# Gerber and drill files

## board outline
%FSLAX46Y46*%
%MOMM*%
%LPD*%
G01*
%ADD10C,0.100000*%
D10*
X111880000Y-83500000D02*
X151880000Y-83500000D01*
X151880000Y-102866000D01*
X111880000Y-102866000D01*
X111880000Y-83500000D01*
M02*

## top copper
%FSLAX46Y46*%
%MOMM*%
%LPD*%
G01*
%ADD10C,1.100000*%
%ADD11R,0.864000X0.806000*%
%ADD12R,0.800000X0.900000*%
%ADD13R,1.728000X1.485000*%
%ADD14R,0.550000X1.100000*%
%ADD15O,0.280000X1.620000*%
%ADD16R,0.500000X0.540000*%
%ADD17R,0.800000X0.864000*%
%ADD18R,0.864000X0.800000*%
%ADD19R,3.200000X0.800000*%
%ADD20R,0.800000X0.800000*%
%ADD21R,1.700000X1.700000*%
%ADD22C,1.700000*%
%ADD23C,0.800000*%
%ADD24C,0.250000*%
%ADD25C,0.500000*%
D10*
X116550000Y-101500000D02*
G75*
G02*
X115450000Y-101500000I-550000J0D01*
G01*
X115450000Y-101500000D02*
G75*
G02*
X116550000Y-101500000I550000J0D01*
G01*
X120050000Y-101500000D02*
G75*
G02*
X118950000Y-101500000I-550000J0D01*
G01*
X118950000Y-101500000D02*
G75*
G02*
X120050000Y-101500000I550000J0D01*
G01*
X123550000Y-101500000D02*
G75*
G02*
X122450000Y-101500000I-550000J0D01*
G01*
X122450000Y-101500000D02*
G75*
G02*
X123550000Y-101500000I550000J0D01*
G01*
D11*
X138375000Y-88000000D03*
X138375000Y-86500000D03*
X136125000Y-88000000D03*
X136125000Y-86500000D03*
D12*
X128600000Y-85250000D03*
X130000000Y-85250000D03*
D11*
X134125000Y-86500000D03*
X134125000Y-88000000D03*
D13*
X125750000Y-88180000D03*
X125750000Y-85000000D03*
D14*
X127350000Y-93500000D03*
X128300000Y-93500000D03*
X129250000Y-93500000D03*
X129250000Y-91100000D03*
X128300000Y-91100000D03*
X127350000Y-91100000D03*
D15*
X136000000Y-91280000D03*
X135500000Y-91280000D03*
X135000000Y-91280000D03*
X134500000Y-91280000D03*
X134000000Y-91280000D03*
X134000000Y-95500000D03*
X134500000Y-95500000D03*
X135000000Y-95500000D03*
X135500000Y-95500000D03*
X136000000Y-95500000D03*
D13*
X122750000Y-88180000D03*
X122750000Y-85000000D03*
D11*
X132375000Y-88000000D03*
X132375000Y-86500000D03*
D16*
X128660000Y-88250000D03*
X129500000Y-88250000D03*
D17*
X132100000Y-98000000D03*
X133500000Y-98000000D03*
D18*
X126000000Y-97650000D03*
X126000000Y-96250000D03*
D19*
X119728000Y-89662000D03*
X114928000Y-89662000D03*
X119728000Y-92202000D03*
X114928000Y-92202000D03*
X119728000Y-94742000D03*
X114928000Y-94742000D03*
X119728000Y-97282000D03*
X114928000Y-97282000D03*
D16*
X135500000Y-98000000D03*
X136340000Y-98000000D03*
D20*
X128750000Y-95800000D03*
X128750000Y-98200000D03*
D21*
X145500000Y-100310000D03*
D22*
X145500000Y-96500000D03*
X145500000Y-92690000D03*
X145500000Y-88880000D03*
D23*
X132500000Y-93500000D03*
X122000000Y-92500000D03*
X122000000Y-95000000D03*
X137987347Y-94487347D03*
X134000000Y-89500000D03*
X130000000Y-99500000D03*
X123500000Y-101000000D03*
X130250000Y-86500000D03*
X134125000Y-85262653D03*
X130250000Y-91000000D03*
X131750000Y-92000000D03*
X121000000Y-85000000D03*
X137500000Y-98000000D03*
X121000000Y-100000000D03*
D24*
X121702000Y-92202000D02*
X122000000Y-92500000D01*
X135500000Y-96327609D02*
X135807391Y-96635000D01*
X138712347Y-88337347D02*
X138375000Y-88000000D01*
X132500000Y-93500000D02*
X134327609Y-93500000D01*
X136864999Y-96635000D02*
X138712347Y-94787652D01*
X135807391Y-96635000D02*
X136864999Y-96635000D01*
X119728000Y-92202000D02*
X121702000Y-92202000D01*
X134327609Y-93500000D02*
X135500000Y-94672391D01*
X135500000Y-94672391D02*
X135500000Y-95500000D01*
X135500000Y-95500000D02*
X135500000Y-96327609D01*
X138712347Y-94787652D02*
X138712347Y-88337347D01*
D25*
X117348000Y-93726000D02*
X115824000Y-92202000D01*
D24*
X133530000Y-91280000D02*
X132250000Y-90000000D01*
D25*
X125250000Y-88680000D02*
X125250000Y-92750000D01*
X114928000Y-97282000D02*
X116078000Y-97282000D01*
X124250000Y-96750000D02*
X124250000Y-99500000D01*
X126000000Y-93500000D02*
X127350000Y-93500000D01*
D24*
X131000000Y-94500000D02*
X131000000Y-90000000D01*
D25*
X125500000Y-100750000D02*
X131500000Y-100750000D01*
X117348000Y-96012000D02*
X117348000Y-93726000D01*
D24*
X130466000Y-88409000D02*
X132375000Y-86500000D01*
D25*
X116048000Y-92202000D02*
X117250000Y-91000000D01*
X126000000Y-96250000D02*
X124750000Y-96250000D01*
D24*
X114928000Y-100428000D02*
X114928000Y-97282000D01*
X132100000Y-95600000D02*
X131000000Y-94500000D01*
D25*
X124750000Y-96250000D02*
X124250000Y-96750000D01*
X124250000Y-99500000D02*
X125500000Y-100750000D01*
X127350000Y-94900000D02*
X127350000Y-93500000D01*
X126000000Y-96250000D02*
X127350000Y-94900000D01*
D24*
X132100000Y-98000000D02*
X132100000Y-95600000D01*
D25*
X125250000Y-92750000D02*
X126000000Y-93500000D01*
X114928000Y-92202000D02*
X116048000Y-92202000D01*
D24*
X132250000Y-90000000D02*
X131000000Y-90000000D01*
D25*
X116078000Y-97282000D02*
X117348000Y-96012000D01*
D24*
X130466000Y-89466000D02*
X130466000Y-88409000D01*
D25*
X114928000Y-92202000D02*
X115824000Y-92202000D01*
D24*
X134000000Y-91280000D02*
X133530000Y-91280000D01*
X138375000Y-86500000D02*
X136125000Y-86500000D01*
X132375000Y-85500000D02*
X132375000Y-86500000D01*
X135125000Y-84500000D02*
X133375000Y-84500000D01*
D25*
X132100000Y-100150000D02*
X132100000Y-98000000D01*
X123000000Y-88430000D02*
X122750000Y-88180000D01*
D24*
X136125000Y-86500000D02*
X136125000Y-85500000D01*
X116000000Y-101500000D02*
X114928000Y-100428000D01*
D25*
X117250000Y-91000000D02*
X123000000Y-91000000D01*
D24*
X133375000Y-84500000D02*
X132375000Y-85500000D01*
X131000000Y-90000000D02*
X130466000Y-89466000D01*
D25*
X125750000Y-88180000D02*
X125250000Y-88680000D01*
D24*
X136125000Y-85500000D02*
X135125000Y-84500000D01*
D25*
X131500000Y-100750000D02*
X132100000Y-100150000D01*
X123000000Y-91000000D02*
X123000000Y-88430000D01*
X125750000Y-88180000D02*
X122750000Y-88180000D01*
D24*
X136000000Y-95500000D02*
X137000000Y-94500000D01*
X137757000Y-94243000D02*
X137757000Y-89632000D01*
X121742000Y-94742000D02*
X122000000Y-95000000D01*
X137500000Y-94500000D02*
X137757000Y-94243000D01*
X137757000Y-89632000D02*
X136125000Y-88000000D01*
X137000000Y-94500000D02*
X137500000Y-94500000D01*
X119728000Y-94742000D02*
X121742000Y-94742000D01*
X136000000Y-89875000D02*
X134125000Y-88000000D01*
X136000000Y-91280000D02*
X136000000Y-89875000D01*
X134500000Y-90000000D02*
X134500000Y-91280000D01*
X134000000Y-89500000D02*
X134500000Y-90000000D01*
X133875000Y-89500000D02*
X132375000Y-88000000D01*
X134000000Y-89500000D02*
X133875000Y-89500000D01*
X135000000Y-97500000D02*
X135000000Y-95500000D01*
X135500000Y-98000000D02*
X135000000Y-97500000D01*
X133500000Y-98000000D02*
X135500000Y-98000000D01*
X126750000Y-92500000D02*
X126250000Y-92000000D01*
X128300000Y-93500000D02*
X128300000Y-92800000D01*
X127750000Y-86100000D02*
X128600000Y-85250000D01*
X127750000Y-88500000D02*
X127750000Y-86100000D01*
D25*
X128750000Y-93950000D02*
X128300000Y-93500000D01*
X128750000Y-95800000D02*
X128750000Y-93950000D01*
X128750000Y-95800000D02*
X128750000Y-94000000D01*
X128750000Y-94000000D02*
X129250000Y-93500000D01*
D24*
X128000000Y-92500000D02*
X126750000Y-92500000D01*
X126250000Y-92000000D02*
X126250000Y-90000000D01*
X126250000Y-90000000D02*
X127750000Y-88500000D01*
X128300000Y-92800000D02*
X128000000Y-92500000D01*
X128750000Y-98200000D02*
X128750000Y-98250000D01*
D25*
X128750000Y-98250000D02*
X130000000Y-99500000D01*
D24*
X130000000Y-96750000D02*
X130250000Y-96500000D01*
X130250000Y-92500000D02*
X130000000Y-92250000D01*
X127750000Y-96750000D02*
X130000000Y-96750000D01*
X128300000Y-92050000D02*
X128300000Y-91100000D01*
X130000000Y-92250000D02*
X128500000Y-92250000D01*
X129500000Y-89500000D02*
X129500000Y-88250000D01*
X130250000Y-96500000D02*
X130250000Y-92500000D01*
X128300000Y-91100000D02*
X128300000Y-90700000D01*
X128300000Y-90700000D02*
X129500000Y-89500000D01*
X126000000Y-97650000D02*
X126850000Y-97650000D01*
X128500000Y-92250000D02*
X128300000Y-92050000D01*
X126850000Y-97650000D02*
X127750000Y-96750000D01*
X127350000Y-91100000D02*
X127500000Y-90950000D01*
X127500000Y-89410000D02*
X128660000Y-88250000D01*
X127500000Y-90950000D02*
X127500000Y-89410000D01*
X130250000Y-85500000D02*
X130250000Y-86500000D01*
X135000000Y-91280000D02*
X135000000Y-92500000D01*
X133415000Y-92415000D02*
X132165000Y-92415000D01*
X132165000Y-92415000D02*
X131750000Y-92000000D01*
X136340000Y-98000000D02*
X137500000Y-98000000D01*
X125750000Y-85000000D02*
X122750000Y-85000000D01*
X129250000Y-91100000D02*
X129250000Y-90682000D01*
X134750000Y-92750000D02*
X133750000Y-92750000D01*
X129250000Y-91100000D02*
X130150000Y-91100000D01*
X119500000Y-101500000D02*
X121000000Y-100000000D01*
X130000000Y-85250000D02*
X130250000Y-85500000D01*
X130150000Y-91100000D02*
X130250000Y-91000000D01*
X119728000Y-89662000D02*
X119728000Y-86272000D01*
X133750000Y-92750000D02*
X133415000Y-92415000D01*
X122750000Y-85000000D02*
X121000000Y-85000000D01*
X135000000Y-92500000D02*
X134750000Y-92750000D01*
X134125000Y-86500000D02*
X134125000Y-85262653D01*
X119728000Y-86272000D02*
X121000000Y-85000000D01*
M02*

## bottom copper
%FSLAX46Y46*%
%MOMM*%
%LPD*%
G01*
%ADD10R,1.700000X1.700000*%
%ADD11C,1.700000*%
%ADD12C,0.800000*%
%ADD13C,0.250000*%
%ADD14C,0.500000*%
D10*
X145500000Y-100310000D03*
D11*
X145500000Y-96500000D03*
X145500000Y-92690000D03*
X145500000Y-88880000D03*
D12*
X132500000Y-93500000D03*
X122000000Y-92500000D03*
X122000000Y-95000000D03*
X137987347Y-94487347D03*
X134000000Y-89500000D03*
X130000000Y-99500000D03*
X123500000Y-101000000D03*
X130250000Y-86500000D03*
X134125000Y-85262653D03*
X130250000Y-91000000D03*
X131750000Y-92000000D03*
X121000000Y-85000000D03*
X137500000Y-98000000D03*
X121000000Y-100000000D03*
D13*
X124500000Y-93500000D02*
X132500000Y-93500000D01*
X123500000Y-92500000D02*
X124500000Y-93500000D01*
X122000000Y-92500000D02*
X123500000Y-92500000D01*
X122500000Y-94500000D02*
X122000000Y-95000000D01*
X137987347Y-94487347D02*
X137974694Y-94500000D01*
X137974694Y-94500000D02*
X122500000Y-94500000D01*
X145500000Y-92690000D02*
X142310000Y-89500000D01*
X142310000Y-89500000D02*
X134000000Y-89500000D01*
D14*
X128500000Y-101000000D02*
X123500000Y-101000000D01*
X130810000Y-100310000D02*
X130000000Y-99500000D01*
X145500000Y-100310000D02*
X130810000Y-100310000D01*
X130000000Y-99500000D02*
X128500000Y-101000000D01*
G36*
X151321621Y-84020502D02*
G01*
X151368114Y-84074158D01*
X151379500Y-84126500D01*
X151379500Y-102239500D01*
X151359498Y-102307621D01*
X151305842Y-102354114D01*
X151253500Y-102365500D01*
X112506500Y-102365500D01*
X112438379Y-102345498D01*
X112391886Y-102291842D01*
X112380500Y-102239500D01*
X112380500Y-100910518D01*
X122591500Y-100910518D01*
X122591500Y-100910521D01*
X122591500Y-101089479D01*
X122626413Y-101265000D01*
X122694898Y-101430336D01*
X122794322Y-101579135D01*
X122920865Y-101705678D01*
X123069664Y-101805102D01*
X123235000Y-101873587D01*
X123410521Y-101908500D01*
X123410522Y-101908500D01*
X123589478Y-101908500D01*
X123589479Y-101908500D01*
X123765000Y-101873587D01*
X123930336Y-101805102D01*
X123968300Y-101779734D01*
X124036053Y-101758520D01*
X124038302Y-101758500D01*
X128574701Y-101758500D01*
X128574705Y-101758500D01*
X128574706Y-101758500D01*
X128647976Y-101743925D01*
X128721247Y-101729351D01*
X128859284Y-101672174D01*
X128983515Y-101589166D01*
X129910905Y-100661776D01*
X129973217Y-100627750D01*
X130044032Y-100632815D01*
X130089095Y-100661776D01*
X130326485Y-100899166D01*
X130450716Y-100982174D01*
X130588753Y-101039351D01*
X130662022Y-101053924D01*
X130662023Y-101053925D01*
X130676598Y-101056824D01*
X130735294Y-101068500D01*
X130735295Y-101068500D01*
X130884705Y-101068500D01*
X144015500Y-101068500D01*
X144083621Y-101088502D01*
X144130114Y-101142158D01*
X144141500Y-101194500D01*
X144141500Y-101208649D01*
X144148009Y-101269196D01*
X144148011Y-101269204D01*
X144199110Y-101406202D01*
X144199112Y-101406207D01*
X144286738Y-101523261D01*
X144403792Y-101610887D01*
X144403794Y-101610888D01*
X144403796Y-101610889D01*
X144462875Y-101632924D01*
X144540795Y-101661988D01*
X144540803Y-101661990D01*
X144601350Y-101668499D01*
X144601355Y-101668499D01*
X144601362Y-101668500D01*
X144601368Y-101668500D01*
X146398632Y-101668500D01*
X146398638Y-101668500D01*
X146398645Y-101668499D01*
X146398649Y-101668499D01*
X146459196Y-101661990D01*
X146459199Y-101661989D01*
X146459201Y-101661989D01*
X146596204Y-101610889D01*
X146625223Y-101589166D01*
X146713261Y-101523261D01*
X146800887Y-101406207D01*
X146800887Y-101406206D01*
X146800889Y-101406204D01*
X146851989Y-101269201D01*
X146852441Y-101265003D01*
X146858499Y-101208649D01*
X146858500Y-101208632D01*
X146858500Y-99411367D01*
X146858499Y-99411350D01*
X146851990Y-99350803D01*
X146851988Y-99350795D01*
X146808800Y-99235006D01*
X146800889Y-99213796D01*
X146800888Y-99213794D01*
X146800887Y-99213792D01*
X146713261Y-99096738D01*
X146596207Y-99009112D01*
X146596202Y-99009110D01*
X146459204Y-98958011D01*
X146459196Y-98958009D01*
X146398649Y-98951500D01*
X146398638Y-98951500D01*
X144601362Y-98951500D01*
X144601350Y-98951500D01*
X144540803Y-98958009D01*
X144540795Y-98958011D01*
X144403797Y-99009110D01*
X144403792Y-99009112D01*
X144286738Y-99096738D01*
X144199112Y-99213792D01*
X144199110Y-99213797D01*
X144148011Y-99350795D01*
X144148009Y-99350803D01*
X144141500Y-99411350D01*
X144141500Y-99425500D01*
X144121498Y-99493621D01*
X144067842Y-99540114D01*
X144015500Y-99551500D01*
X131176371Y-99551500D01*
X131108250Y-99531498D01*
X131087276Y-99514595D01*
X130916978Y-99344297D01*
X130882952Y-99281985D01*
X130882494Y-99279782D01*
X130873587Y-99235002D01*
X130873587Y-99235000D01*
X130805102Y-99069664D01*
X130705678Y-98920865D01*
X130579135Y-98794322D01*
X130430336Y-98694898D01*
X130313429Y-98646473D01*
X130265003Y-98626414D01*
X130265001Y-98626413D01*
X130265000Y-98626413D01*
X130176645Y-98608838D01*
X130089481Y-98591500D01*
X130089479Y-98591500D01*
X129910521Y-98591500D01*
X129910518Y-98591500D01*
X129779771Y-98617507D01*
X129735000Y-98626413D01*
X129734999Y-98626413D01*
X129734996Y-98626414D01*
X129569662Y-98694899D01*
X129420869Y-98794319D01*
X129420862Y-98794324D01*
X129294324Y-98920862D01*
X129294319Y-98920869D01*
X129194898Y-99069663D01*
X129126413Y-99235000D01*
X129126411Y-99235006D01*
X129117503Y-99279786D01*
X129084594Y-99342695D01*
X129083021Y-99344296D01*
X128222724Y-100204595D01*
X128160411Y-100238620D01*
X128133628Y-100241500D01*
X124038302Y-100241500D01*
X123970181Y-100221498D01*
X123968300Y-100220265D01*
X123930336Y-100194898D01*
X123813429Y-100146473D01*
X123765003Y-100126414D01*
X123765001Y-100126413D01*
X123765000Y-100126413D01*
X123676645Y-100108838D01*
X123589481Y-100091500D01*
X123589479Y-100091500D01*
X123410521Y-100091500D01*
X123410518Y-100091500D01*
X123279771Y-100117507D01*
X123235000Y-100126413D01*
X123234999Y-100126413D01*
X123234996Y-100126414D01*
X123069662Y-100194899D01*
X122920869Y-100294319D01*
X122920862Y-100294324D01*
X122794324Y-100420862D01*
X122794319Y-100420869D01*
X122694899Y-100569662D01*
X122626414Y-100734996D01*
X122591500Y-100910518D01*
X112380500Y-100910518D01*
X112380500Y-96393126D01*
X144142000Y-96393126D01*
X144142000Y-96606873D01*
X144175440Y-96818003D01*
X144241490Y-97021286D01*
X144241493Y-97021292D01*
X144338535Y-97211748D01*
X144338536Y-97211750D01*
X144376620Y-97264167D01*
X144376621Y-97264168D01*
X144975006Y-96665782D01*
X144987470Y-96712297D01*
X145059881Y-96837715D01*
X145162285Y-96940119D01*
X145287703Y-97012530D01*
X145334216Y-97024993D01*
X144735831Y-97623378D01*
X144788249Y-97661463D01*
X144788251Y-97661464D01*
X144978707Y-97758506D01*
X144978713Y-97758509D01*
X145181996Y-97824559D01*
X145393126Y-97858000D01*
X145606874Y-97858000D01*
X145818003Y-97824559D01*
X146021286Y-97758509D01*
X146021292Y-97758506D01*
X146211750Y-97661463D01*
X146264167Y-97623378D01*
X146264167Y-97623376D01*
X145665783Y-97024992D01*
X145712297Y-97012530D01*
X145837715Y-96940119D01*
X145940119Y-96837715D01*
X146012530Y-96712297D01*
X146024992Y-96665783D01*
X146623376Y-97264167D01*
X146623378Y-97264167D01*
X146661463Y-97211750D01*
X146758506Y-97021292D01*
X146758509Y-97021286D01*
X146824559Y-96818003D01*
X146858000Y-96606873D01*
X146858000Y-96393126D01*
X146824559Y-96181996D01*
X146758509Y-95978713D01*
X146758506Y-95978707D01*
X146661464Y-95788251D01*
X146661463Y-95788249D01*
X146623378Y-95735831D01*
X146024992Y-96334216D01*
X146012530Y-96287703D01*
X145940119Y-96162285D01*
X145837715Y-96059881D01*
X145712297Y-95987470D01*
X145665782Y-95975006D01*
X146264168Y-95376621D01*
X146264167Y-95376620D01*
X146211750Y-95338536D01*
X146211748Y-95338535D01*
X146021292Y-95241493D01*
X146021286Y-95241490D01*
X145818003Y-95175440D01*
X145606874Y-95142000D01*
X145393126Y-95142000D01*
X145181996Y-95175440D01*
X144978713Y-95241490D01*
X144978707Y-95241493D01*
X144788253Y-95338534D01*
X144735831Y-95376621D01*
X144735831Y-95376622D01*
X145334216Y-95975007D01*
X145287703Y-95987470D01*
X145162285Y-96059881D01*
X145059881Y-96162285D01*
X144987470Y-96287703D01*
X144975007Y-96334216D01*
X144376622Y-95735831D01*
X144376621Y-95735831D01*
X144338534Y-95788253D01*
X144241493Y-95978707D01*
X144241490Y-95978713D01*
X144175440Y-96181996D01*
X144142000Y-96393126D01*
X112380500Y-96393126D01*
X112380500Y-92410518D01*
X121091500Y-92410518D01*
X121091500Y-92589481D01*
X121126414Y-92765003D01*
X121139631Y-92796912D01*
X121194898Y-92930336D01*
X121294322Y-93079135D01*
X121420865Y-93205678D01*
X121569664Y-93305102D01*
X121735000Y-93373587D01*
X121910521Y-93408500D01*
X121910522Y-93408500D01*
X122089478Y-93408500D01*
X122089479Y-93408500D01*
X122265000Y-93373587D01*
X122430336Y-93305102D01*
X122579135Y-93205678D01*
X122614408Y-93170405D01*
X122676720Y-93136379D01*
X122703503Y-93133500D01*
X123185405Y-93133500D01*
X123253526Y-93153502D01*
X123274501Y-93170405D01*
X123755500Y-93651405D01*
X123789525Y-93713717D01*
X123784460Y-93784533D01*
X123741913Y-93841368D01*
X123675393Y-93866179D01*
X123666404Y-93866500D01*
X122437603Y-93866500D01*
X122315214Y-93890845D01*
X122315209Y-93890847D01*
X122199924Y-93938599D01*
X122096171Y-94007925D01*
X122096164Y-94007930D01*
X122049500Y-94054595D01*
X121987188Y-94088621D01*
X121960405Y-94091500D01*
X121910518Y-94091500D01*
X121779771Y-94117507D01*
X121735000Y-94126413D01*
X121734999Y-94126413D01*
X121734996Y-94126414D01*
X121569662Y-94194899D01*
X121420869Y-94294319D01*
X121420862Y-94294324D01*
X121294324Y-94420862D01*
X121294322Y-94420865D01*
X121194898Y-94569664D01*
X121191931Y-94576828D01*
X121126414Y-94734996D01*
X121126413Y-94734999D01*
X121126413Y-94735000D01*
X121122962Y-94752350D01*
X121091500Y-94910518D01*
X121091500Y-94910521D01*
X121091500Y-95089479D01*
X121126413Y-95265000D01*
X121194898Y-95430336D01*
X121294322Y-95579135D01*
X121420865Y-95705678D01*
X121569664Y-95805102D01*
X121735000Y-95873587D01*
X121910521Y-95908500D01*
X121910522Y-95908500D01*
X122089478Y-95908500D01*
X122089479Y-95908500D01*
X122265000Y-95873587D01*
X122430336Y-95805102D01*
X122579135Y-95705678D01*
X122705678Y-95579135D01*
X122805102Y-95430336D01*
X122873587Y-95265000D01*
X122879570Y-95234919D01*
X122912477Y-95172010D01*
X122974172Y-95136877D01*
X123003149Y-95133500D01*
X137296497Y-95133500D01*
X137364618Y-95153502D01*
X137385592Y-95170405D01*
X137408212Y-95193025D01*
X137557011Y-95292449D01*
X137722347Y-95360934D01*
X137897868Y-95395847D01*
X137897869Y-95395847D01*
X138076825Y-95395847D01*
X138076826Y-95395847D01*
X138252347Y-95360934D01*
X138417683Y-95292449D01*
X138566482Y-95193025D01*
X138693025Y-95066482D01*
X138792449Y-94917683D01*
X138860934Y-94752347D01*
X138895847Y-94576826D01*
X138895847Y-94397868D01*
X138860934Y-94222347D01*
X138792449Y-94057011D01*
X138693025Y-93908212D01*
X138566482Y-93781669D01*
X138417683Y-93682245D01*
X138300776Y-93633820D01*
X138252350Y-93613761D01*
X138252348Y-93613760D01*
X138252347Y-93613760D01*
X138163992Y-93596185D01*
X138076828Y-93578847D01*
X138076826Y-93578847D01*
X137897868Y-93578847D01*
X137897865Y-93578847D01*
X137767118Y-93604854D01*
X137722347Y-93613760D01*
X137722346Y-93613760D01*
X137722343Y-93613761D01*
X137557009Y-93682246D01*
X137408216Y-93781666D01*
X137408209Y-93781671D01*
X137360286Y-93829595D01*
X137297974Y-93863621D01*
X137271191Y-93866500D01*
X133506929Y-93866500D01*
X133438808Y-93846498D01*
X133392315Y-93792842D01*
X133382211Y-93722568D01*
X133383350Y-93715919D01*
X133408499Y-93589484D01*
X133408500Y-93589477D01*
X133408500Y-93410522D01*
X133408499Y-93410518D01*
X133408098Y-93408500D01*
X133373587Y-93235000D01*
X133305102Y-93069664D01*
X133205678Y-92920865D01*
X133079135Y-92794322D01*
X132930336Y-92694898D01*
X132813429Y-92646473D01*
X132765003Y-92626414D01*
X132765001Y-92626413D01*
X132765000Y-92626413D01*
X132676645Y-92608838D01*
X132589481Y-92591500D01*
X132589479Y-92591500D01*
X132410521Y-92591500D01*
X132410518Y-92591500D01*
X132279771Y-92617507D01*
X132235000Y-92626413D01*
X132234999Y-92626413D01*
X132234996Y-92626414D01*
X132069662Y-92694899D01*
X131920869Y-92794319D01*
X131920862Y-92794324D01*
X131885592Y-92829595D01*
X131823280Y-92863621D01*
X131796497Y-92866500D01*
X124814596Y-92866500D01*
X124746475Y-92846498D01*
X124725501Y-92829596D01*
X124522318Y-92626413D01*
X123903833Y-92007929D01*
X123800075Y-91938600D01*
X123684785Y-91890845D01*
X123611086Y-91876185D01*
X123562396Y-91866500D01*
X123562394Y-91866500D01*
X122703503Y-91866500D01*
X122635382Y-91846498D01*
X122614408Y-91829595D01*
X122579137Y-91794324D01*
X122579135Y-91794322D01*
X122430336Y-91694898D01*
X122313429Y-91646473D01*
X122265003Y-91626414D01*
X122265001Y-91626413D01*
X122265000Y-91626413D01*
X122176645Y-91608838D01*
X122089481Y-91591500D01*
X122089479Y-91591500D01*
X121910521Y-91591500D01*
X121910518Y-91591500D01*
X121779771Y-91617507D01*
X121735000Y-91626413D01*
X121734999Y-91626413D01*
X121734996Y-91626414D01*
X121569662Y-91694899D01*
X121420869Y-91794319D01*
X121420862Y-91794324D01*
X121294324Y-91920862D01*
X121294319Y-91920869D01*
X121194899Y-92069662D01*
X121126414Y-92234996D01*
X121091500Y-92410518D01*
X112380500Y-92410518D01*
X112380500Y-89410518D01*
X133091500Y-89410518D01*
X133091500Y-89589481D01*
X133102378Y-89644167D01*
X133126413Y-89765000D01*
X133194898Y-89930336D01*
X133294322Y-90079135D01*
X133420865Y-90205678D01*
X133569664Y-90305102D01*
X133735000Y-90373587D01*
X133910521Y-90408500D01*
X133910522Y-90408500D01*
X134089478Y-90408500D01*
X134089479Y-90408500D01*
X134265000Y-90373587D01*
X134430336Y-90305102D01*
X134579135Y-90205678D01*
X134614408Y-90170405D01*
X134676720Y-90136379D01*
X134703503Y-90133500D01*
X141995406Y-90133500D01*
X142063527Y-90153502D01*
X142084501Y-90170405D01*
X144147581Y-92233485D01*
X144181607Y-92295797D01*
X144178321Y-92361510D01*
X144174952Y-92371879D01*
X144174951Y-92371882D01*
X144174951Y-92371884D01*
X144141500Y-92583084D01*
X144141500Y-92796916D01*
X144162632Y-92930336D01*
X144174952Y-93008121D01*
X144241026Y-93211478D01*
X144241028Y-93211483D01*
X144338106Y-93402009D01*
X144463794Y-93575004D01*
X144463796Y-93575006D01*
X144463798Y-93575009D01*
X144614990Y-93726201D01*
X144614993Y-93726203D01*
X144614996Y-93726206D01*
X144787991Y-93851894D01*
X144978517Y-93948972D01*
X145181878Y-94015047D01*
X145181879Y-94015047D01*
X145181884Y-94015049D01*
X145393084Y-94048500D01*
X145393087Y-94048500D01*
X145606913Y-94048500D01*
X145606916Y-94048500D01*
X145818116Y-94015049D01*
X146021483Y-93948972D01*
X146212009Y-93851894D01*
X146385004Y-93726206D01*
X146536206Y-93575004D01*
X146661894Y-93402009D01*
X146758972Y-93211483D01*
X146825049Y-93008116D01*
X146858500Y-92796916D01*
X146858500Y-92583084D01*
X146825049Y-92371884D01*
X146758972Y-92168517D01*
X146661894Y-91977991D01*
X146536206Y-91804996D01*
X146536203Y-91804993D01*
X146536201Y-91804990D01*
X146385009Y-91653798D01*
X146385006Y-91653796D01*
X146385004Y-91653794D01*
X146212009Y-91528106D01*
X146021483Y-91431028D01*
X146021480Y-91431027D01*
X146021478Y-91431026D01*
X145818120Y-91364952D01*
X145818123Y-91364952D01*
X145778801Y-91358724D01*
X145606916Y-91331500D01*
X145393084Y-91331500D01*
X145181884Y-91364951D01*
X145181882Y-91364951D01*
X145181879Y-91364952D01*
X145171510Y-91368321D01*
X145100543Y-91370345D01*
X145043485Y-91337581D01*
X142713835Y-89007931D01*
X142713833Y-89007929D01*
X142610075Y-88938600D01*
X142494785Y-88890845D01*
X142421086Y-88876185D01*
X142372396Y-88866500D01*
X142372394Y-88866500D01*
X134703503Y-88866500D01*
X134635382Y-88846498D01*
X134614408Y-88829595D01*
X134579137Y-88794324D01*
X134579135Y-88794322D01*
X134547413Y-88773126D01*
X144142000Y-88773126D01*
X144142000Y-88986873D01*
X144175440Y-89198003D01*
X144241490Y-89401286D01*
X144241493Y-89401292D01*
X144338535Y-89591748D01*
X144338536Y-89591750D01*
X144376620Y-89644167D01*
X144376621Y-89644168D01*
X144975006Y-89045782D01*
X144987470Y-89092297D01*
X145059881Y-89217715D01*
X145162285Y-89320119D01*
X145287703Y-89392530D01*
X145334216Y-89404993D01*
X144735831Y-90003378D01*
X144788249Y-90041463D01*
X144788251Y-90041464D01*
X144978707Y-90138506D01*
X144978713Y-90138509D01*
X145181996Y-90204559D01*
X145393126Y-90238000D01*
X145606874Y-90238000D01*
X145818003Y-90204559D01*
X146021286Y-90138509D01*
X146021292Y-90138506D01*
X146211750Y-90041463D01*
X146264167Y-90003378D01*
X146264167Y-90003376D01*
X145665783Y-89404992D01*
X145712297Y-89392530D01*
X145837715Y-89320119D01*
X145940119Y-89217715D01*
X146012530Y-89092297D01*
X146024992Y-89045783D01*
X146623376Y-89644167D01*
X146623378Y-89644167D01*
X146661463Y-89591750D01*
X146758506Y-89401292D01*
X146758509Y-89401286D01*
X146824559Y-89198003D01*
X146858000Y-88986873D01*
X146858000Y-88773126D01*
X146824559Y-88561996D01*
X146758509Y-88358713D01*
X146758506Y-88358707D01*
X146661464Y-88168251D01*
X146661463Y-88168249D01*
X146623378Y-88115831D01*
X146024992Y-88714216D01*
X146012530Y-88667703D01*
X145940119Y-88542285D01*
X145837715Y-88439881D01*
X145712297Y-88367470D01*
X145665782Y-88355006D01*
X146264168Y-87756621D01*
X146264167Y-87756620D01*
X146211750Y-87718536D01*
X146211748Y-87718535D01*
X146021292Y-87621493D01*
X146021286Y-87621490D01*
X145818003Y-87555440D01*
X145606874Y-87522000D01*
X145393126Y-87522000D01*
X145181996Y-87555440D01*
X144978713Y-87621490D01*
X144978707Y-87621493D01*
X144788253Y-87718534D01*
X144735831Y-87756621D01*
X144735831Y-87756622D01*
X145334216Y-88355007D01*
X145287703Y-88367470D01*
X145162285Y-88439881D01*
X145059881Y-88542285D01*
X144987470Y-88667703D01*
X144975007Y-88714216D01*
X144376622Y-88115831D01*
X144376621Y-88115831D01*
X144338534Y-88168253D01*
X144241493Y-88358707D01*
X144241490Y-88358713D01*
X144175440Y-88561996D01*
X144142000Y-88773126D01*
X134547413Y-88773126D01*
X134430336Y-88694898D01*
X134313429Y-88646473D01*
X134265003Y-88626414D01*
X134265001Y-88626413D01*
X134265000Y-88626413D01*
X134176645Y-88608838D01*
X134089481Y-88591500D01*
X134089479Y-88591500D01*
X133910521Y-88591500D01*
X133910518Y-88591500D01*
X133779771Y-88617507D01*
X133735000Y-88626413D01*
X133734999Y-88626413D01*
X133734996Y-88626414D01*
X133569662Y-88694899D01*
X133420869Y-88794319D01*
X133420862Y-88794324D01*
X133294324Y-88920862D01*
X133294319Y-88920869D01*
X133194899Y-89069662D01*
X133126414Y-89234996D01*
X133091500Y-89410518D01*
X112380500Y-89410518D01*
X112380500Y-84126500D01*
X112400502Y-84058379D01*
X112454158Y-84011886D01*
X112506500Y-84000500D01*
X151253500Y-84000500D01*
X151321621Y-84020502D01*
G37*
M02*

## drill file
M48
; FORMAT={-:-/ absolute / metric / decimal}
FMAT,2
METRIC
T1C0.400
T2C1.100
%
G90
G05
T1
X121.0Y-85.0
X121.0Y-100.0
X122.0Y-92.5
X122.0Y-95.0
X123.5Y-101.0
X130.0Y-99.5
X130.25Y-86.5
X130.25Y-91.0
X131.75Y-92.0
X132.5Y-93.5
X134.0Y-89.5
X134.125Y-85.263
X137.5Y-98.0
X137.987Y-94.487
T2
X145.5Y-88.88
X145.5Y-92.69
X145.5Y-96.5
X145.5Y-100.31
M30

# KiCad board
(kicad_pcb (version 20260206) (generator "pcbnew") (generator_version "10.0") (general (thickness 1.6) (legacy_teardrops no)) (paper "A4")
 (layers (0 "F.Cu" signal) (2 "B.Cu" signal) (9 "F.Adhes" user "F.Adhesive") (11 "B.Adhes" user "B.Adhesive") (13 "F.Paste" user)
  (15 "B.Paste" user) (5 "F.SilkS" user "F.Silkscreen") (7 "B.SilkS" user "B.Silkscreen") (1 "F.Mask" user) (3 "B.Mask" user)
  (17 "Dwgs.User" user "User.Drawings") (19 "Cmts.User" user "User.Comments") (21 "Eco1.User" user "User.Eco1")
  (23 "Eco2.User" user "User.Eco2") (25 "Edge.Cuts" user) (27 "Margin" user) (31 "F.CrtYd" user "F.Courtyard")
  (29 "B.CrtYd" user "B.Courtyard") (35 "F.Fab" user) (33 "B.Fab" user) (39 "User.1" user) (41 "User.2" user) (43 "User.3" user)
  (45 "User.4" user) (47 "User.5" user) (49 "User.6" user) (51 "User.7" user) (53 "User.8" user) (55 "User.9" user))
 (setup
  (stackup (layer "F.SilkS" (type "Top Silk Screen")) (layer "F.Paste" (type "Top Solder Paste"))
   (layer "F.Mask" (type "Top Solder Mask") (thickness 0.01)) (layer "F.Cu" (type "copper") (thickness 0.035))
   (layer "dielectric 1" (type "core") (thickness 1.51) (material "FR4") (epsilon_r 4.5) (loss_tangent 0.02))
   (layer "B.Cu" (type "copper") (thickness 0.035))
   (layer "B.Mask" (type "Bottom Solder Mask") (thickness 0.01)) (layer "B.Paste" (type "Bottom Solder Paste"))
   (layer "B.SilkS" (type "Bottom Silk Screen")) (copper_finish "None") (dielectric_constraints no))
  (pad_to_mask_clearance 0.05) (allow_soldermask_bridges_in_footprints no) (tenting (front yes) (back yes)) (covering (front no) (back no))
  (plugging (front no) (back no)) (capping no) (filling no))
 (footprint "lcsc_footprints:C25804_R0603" (layer "F.Cu") (at 138.375 87.25 90)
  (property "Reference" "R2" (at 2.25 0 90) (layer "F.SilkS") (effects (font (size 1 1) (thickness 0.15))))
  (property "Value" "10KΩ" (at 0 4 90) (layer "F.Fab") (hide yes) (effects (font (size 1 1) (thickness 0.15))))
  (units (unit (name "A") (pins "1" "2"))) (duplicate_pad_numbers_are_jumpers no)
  (pad "1" smd rect (at -0.75 0 90) (size 0.806 0.864) (layers "F.Cu" "F.Mask" "F.Paste") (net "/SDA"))
  (pad "2" smd rect (at 0.75 0 90) (size 0.806 0.864) (layers "F.Cu" "F.Mask" "F.Paste") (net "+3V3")))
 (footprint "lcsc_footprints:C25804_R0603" (layer "F.Cu") (at 136.125 87.25 90)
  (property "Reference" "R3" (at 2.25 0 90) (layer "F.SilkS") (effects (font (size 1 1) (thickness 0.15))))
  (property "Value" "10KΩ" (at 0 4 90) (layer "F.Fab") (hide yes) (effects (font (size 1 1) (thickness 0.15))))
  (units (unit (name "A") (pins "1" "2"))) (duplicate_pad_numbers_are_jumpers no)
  (pad "1" smd rect (at -0.75 0 90) (size 0.806 0.864) (layers "F.Cu" "F.Mask" "F.Paste") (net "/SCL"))
  (pad "2" smd rect (at 0.75 0 90) (size 0.806 0.864) (layers "F.Cu" "F.Mask" "F.Paste") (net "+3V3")))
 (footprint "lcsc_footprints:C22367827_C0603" (layer "F.Cu") (at 129.3 85.25)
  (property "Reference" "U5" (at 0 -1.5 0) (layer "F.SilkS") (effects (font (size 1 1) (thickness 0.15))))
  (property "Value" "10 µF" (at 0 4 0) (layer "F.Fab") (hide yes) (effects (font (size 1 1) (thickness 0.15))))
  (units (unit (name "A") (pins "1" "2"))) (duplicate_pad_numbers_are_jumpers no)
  (pad "1" smd rect (at -0.7 0) (size 0.8 0.9) (layers "F.Cu" "F.Mask" "F.Paste") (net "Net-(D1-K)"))
  (pad "2" smd rect (at 0.7 0) (size 0.8 0.9) (layers "F.Cu" "F.Mask" "F.Paste") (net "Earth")))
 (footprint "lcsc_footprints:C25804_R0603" (layer "F.Cu") (at 134.125 87.25 -90)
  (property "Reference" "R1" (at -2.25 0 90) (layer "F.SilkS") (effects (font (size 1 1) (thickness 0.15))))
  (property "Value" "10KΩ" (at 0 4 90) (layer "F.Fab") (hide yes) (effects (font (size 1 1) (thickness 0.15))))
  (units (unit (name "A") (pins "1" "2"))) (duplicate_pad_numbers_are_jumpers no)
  (pad "1" smd rect (at -0.75 0 270) (size 0.806 0.864) (layers "F.Cu" "F.Mask" "F.Paste") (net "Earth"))
  (pad "2" smd rect (at 0.75 0 270) (size 0.806 0.864) (layers "F.Cu" "F.Mask" "F.Paste") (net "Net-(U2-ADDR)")))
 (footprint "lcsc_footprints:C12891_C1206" (layer "F.Cu") (at 125.75 86.59 90)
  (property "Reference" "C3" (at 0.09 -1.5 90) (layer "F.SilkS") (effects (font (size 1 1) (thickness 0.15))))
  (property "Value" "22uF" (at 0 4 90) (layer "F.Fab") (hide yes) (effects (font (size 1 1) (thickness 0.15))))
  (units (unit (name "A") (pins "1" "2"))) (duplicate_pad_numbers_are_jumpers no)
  (pad "1" smd rect (at -1.59 0 90) (size 1.485 1.728) (layers "F.Cu" "F.Mask" "F.Paste") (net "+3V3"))
  (pad "2" smd rect (at 1.59 0 90) (size 1.485 1.728) (layers "F.Cu" "F.Mask" "F.Paste") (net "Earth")))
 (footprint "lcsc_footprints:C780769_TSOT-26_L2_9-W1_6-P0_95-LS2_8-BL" (layer "F.Cu") (at 128.3 92.3)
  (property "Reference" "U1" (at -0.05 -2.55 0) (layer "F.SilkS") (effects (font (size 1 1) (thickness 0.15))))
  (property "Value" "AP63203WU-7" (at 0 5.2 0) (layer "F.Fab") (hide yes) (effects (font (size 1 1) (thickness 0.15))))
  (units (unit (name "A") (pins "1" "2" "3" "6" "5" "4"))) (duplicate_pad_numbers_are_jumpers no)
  (pad "1" smd rect (at -0.95 1.2 180) (size 0.55 1.1) (layers "F.Cu" "F.Mask" "F.Paste") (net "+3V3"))
  (pad "2" smd rect (at 0 1.2 180) (size 0.55 1.1) (layers "F.Cu" "F.Mask" "F.Paste") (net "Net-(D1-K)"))
  (pad "3" smd rect (at 0.95 1.2 180) (size 0.55 1.1) (layers "F.Cu" "F.Mask" "F.Paste") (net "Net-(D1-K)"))
  (pad "4" smd rect (at 0.95 -1.2 180) (size 0.55 1.1) (layers "F.Cu" "F.Mask" "F.Paste") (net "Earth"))
  (pad "5" smd rect (at 0 -1.2 180) (size 0.55 1.1) (layers "F.Cu" "F.Mask" "F.Paste") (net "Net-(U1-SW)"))
  (pad "6" smd rect (at -0.95 -1.2 180) (size 0.55 1.1) (layers "F.Cu" "F.Mask" "F.Paste") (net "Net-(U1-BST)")))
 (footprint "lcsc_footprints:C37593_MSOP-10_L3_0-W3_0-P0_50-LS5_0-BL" (layer "F.Cu") (at 135 93.39 180)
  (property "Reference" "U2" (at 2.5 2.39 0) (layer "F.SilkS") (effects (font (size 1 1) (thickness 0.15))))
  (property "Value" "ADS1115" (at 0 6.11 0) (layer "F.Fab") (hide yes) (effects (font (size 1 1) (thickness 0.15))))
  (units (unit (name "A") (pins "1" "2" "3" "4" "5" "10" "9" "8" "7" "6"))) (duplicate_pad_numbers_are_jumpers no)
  (pad "1" smd oval (at -1 2.11 180) (size 0.28 1.62) (layers "F.Cu" "F.Mask" "F.Paste") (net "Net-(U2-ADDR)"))
  (pad "2" smd oval (at -0.5 2.11 180) (size 0.28 1.62) (layers "F.Cu" "F.Mask" "F.Paste") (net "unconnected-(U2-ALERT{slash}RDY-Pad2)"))
  (pad "3" smd oval (at 0 2.11 180) (size 0.28 1.62) (layers "F.Cu" "F.Mask" "F.Paste") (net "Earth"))
  (pad "4" smd oval (at 0.5 2.11 180) (size 0.28 1.62) (layers "F.Cu" "F.Mask" "F.Paste") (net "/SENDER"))
  (pad "5" smd oval (at 1 2.11 180) (size 0.28 1.62) (layers "F.Cu" "F.Mask" "F.Paste") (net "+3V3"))
  (pad "6" smd oval (at 1 -2.11 180) (size 0.28 1.62) (layers "F.Cu" "F.Mask" "F.Paste") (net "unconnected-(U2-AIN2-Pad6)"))
  (pad "7" smd oval (at 0.5 -2.11 180) (size 0.28 1.62) (layers "F.Cu" "F.Mask" "F.Paste") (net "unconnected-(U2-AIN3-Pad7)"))
  (pad "8" smd oval (at 0 -2.11 180) (size 0.28 1.62) (layers "F.Cu" "F.Mask" "F.Paste") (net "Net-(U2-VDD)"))
  (pad "9" smd oval (at -0.5 -2.11 180) (size 0.28 1.62) (layers "F.Cu" "F.Mask" "F.Paste") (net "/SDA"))
  (pad "10" smd oval (at -1 -2.11 180) (size 0.28 1.62) (layers "F.Cu" "F.Mask" "F.Paste") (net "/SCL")))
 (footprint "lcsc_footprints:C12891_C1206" (layer "F.Cu") (at 122.75 86.59 90)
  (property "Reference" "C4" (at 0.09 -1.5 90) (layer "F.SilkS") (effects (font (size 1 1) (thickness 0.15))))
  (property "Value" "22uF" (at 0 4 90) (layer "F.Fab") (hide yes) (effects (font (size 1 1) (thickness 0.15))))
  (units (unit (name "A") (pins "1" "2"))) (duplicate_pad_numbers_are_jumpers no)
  (pad "1" smd rect (at -1.59 0 90) (size 1.485 1.728) (layers "F.Cu" "F.Mask" "F.Paste") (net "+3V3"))
  (pad "2" smd rect (at 1.59 0 90) (size 1.485 1.728) (layers "F.Cu" "F.Mask" "F.Paste") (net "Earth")))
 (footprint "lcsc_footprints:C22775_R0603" (layer "F.Cu") (at 132.375 87.25 90)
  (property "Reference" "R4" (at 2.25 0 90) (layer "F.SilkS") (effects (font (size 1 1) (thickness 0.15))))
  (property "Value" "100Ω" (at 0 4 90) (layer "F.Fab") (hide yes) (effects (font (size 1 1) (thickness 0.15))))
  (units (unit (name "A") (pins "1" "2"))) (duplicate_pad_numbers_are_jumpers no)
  (pad "1" smd rect (at -0.75 0 90) (size 0.806 0.864) (layers "F.Cu" "F.Mask" "F.Paste") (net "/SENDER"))
  (pad "2" smd rect (at 0.75 0 90) (size 0.806 0.864) (layers "F.Cu" "F.Mask" "F.Paste") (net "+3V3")))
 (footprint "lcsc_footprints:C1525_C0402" (layer "F.Cu") (at 129.08 88.25)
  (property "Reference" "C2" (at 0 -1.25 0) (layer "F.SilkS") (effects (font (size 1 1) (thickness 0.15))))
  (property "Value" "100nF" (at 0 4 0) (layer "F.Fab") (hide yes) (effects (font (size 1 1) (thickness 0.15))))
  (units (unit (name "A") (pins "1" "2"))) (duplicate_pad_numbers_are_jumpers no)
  (pad "1" smd rect (at -0.42 0) (size 0.5 0.54) (layers "F.Cu" "F.Mask" "F.Paste") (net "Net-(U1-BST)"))
  (pad "2" smd rect (at 0.42 0) (size 0.5 0.54) (layers "F.Cu" "F.Mask" "F.Paste") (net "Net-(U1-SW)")))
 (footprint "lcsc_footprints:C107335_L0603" (layer "F.Cu") (at 132.8 98)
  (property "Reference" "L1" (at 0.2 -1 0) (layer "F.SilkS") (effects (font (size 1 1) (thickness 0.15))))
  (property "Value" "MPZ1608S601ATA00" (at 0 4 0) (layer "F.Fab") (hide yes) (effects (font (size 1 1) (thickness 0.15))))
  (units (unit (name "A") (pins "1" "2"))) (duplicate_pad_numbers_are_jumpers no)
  (pad "1" smd rect (at -0.7 0 180) (size 0.8 0.864) (layers "F.Cu" "F.Mask" "F.Paste") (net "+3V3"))
  (pad "2" smd rect (at 0.7 0 180) (size 0.8 0.864) (layers "F.Cu" "F.Mask" "F.Paste") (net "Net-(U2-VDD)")))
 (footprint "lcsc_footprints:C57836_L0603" (layer "F.Cu") (at 126 96.95 90)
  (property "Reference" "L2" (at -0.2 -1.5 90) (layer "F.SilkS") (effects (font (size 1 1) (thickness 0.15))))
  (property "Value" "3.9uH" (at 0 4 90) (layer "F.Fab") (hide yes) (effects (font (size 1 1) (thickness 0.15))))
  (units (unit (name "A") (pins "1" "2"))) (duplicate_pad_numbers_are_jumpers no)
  (pad "1" smd rect (at -0.7 0 270) (size 0.8 0.864) (layers "F.Cu" "F.Mask" "F.Paste") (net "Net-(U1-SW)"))
  (pad "2" smd rect (at 0.7 0 270) (size 0.8 0.864) (layers "F.Cu" "F.Mask" "F.Paste") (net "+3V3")))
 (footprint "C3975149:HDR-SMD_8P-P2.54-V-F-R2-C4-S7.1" (layer "F.Cu") (at 117.328 93.472 -90)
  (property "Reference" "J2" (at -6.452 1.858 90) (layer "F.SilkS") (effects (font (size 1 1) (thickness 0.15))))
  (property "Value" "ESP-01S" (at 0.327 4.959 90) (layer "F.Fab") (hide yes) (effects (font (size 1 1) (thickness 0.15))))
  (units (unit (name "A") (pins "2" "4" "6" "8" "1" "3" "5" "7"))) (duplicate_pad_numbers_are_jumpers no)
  (pad "1" smd rect (at -3.81 -2.4 270) (size 0.8 3.2) (layers "F.Cu" "F.Mask" "F.Paste") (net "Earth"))
  (pad "2" smd rect (at -3.81 2.4 270) (size 0.8 3.2) (layers "F.Cu" "F.Mask" "F.Paste") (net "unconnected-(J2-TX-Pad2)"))
  (pad "3" smd rect (at -1.27 -2.4 270) (size 0.8 3.2) (layers "F.Cu" "F.Mask" "F.Paste") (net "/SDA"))
  (pad "4" smd rect (at -1.27 2.4 270) (size 0.8 3.2) (layers "F.Cu" "F.Mask" "F.Paste") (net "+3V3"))
  (pad "5" smd rect (at 1.27 -2.4 270) (size 0.8 3.2) (layers "F.Cu" "F.Mask" "F.Paste") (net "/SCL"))
  (pad "6" smd rect (at 1.27 2.4 270) (size 0.8 3.2) (layers "F.Cu" "F.Mask" "F.Paste") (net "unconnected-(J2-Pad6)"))
  (pad "7" smd rect (at 3.81 -2.4 270) (size 0.8 3.2) (layers "F.Cu" "F.Mask" "F.Paste") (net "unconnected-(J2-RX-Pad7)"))
  (pad "8" smd rect (at 3.81 2.4 270) (size 0.8 3.2) (layers "F.Cu" "F.Mask" "F.Paste") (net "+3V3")))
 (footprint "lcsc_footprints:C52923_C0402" (layer "F.Cu") (at 135.92 98)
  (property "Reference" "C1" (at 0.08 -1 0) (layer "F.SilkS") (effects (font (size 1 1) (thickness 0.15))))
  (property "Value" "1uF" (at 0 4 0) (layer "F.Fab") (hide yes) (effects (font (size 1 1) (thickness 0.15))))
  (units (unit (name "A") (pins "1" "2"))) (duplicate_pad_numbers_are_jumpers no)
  (pad "1" smd rect (at -0.42 0) (size 0.5 0.54) (layers "F.Cu" "F.Mask" "F.Paste") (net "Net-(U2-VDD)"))
  (pad "2" smd rect (at 0.42 0) (size 0.5 0.54) (layers "F.Cu" "F.Mask" "F.Paste") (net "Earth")))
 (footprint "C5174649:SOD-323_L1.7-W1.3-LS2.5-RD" (layer "F.Cu") (at 128.75 97 -90)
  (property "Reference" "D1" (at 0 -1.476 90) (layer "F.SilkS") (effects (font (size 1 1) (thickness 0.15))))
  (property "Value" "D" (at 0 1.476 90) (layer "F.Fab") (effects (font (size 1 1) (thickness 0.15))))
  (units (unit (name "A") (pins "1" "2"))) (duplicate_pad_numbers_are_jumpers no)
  (pad "1" smd rect (at -1.2 0 270) (size 0.8 0.8) (layers "F.Cu" "F.Mask" "F.Paste") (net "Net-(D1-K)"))
  (pad "2" smd rect (at 1.2 0 270) (size 0.8 0.8) (layers "F.Cu" "F.Mask" "F.Paste") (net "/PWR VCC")))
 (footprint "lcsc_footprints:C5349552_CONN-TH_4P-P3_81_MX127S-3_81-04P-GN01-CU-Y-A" (layer "F.Cu") (at 145.5 94.6 90)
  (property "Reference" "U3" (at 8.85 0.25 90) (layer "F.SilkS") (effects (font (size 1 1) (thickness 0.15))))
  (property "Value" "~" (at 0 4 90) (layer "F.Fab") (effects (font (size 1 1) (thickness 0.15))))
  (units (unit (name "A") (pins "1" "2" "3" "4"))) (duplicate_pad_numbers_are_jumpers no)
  (pad "1" thru_hole rect (at -5.71 0 90) (size 1.7 1.7) (drill 1.100024) (layers "*.Cu" "*.Mask") (remove_unused_layers no)
   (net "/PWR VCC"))
  (pad "2" thru_hole circle (at -1.9 0 90) (size 1.7 1.7) (drill 1.100024) (layers "*.Cu" "*.Mask") (remove_unused_layers no) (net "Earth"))
  (pad "3" thru_hole circle (at 1.91 0 90) (size 1.7 1.7) (drill 1.100024) (layers "*.Cu" "*.Mask") (remove_unused_layers no)
   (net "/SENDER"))
  (pad "4" thru_hole circle (at 5.72 0 90) (size 1.7 1.7) (drill 1.100024) (layers "*.Cu" "*.Mask") (remove_unused_layers no) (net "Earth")))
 (gr_circle (center 116 101.5) (end 117 101.5) (stroke (width 0.2) (type solid)) (fill yes) (layer "F.Cu") (net "+3V3"))
 (gr_circle (center 119.5 101.5) (end 120.5 101.5) (stroke (width 0.2) (type solid)) (fill yes) (layer "F.Cu") (net "Earth"))
 (gr_circle (center 123 101.5) (end 124 101.5) (stroke (width 0.2) (type solid)) (fill yes) (layer "F.Cu") (net "/PWR VCC"))
 (gr_rect (start 111.88 83.5) (end 151.88 102.866) (stroke (width 0.1) (type solid)) (fill no) (layer "Edge.Cuts"))
 (segment (start 121.702 92.202) (end 122 92.5) (width 0.25) (layer "F.Cu") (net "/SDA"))
 (segment (start 135.5 96.327609) (end 135.807391 96.635) (width 0.25) (layer "F.Cu") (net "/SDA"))
 (segment (start 138.712347 88.337347) (end 138.375 88) (width 0.25) (layer "F.Cu") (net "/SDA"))
 (segment (start 132.5 93.5) (end 134.327609 93.5) (width 0.25) (layer "F.Cu") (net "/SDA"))
 (segment (start 136.864999 96.635) (end 138.712347 94.787652) (width 0.25) (layer "F.Cu") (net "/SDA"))
 (segment (start 135.807391 96.635) (end 136.864999 96.635) (width 0.25) (layer "F.Cu") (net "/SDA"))
 (segment (start 119.728 92.202) (end 121.702 92.202) (width 0.25) (layer "F.Cu") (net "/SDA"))
 (segment (start 134.327609 93.5) (end 135.5 94.672391) (width 0.25) (layer "F.Cu") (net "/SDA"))
 (segment (start 135.5 94.672391) (end 135.5 95.5) (width 0.25) (layer "F.Cu") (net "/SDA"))
 (segment (start 135.5 95.5) (end 135.5 96.327609) (width 0.25) (layer "F.Cu") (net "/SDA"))
 (segment (start 138.712347 94.787652) (end 138.712347 88.337347) (width 0.25) (layer "F.Cu") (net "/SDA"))
 (via (at 132.5 93.5) (size 0.8) (drill 0.4) (layers "F.Cu" "B.Cu") (free yes) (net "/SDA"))
 (via (at 122 92.5) (size 0.8) (drill 0.4) (layers "F.Cu" "B.Cu") (free yes) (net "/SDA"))
 (segment (start 124.5 93.5) (end 132.5 93.5) (width 0.25) (layer "B.Cu") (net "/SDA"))
 (segment (start 123.5 92.5) (end 124.5 93.5) (width 0.25) (layer "B.Cu") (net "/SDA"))
 (segment (start 122 92.5) (end 123.5 92.5) (width 0.25) (layer "B.Cu") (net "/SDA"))
 (segment (start 117.348 93.726) (end 115.824 92.202) (width 0.5) (layer "F.Cu") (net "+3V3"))
 (segment (start 133.53 91.28) (end 132.25 90) (width 0.25) (layer "F.Cu") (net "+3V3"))
 (segment (start 125.25 88.68) (end 125.25 92.75) (width 0.5) (layer "F.Cu") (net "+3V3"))
 (segment (start 114.928 97.282) (end 116.078 97.282) (width 0.5) (layer "F.Cu") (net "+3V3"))
 (segment (start 124.25 96.75) (end 124.25 99.5) (width 0.5) (layer "F.Cu") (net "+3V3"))
 (segment (start 126 93.5) (end 127.35 93.5) (width 0.5) (layer "F.Cu") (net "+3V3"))
 (segment (start 131 94.5) (end 131 90) (width 0.25) (layer "F.Cu") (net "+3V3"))
 (segment (start 125.5 100.75) (end 131.5 100.75) (width 0.5) (layer "F.Cu") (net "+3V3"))
 (segment (start 117.348 96.012) (end 117.348 93.726) (width 0.5) (layer "F.Cu") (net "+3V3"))
 (segment (start 130.466 88.409) (end 132.375 86.5) (width 0.25) (layer "F.Cu") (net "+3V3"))
 (segment (start 116.048 92.202) (end 117.25 91) (width 0.5) (layer "F.Cu") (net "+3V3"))
 (segment (start 126 96.25) (end 124.75 96.25) (width 0.5) (layer "F.Cu") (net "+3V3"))
 (segment (start 114.928 100.428) (end 114.928 97.282) (width 0.25) (layer "F.Cu") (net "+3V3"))
 (segment (start 132.1 95.6) (end 131 94.5) (width 0.25) (layer "F.Cu") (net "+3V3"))
 (segment (start 124.75 96.25) (end 124.25 96.75) (width 0.5) (layer "F.Cu") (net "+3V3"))
 (segment (start 124.25 99.5) (end 125.5 100.75) (width 0.5) (layer "F.Cu") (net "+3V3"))
 (segment (start 127.35 94.9) (end 127.35 93.5) (width 0.5) (layer "F.Cu") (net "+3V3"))
 (segment (start 126 96.25) (end 127.35 94.9) (width 0.5) (layer "F.Cu") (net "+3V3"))
 (segment (start 132.1 98) (end 132.1 95.6) (width 0.25) (layer "F.Cu") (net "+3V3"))
 (segment (start 125.25 92.75) (end 126 93.5) (width 0.5) (layer "F.Cu") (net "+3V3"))
 (segment (start 114.928 92.202) (end 116.048 92.202) (width 0.5) (layer "F.Cu") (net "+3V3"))
 (segment (start 132.25 90) (end 131 90) (width 0.25) (layer "F.Cu") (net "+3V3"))
 (segment (start 116.078 97.282) (end 117.348 96.012) (width 0.5) (layer "F.Cu") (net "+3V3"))
 (segment (start 130.466 89.466) (end 130.466 88.409) (width 0.25) (layer "F.Cu") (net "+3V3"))
 (segment (start 114.928 92.202) (end 115.824 92.202) (width 0.5) (layer "F.Cu") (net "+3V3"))
 (segment (start 134 91.28) (end 133.53 91.28) (width 0.25) (layer "F.Cu") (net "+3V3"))
 (segment (start 138.375 86.5) (end 136.125 86.5) (width 0.25) (layer "F.Cu") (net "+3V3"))
 (segment (start 132.375 85.5) (end 132.375 86.5) (width 0.25) (layer "F.Cu") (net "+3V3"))
 (segment (start 135.125 84.5) (end 133.375 84.5) (width 0.25) (layer "F.Cu") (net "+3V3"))
 (segment (start 132.1 100.15) (end 132.1 98) (width 0.5) (layer "F.Cu") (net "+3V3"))
 (segment (start 123 88.43) (end 122.75 88.18) (width 0.5) (layer "F.Cu") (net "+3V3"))
 (segment (start 136.125 86.5) (end 136.125 85.5) (width 0.25) (layer "F.Cu") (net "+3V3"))
 (segment (start 116 101.5) (end 114.928 100.428) (width 0.25) (layer "F.Cu") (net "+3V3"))
 (segment (start 117.25 91) (end 123 91) (width 0.5) (layer "F.Cu") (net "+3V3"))
 (segment (start 133.375 84.5) (end 132.375 85.5) (width 0.25) (layer "F.Cu") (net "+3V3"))
 (segment (start 131 90) (end 130.466 89.466) (width 0.25) (layer "F.Cu") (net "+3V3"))
 (segment (start 125.75 88.18) (end 125.25 88.68) (width 0.5) (layer "F.Cu") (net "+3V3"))
 (segment (start 136.125 85.5) (end 135.125 84.5) (width 0.25) (layer "F.Cu") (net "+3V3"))
 (segment (start 131.5 100.75) (end 132.1 100.15) (width 0.5) (layer "F.Cu") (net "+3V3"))
 (segment (start 123 91) (end 123 88.43) (width 0.5) (layer "F.Cu") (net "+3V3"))
 (segment (start 125.75 88.18) (end 122.75 88.18) (width 0.5) (layer "F.Cu") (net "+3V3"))
 (segment (start 136 95.5) (end 137 94.5) (width 0.25) (layer "F.Cu") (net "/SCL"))
 (segment (start 137.757 94.243) (end 137.757 89.632) (width 0.25) (layer "F.Cu") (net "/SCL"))
 (segment (start 121.742 94.742) (end 122 95) (width 0.25) (layer "F.Cu") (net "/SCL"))
 (segment (start 137.5 94.5) (end 137.757 94.243) (width 0.25) (layer "F.Cu") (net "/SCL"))
 (segment (start 137.757 89.632) (end 136.125 88) (width 0.25) (layer "F.Cu") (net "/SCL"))
 (segment (start 137 94.5) (end 137.5 94.5) (width 0.25) (layer "F.Cu") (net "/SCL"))
 (segment (start 119.728 94.742) (end 121.742 94.742) (width 0.25) (layer "F.Cu") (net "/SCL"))
 (via (at 122 95) (size 0.8) (drill 0.4) (layers "F.Cu" "B.Cu") (free yes) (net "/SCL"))
 (via (at 137.987347 94.487347) (size 0.8) (drill 0.4) (layers "F.Cu" "B.Cu") (free yes) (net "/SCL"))
 (segment (start 122.5 94.5) (end 122 95) (width 0.25) (layer "B.Cu") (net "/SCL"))
 (segment (start 137.987347 94.487347) (end 137.974694 94.5) (width 0.25) (layer "B.Cu") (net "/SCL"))
 (segment (start 137.974694 94.5) (end 122.5 94.5) (width 0.25) (layer "B.Cu") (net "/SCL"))
 (segment (start 136 89.875) (end 134.125 88) (width 0.25) (layer "F.Cu") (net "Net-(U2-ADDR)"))
 (segment (start 136 91.28) (end 136 89.875) (width 0.25) (layer "F.Cu") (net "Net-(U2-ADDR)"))
 (segment (start 134.5 90) (end 134.5 91.28) (width 0.25) (layer "F.Cu") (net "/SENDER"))
 (segment (start 134 89.5) (end 134.5 90) (width 0.25) (layer "F.Cu") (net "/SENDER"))
 (segment (start 133.875 89.5) (end 132.375 88) (width 0.25) (layer "F.Cu") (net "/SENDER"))
 (segment (start 134 89.5) (end 133.875 89.5) (width 0.25) (layer "F.Cu") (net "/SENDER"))
 (via (at 134 89.5) (size 0.8) (drill 0.4) (layers "F.Cu" "B.Cu") (free yes) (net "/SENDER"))
 (segment (start 145.5 92.69) (end 142.31 89.5) (width 0.25) (layer "B.Cu") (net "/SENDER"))
 (segment (start 142.31 89.5) (end 134 89.5) (width 0.25) (layer "B.Cu") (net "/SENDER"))
 (segment (start 135 97.5) (end 135 95.5) (width 0.25) (layer "F.Cu") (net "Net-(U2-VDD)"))
 (segment (start 135.5 98) (end 135 97.5) (width 0.25) (layer "F.Cu") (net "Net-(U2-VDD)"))
 (segment (start 133.5 98) (end 135.5 98) (width 0.25) (layer "F.Cu") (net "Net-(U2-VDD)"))
 (segment (start 126.75 92.5) (end 126.25 92) (width 0.25) (layer "F.Cu") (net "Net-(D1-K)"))
 (segment (start 128.3 93.5) (end 128.3 92.8) (width 0.25) (layer "F.Cu") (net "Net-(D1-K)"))
 (segment (start 127.75 86.1) (end 128.6 85.25) (width 0.25) (layer "F.Cu") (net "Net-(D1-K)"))
 (segment (start 127.75 88.5) (end 127.75 86.1) (width 0.25) (layer "F.Cu") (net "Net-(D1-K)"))
 (segment (start 128.75 93.95) (end 128.3 93.5) (width 0.5) (layer "F.Cu") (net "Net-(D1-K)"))
 (segment (start 128.75 95.8) (end 128.75 93.95) (width 0.5) (layer "F.Cu") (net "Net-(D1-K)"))
 (segment (start 128.75 95.8) (end 128.75 94) (width 0.5) (layer "F.Cu") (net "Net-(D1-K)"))
 (segment (start 128.75 94) (end 129.25 93.5) (width 0.5) (layer "F.Cu") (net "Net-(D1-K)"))
 (segment (start 128 92.5) (end 126.75 92.5) (width 0.25) (layer "F.Cu") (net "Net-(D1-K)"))
 (segment (start 126.25 92) (end 126.25 90) (width 0.25) (layer "F.Cu") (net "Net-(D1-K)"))
 (segment (start 126.25 90) (end 127.75 88.5) (width 0.25) (layer "F.Cu") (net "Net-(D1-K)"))
 (segment (start 128.3 92.8) (end 128 92.5) (width 0.25) (layer "F.Cu") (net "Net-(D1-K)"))
 (segment (start 128.75 98.2) (end 128.75 98.25) (width 0.25) (layer "F.Cu") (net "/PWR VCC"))
 (segment (start 128.75 98.25) (end 130 99.5) (width 0.5) (layer "F.Cu") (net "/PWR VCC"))
 (via (at 130 99.5) (size 0.8) (drill 0.4) (layers "F.Cu" "B.Cu") (free yes) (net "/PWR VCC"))
 (via (at 123.5 101) (size 0.8) (drill 0.4) (layers "F.Cu" "B.Cu") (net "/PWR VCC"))
 (segment (start 128.5 101) (end 123.5 101) (width 0.5) (layer "B.Cu") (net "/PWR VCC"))
 (segment (start 130.81 100.31) (end 130 99.5) (width 0.5) (layer "B.Cu") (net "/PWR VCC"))
 (segment (start 145.5 100.31) (end 130.81 100.31) (width 0.5) (layer "B.Cu") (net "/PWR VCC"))
 (segment (start 130 99.5) (end 128.5 101) (width 0.5) (layer "B.Cu") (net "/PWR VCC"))
 (segment (start 130 96.75) (end 130.25 96.5) (width 0.25) (layer "F.Cu") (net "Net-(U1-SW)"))
 (segment (start 130.25 92.5) (end 130 92.25) (width 0.25) (layer "F.Cu") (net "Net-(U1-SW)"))
 (segment (start 127.75 96.75) (end 130 96.75) (width 0.25) (layer "F.Cu") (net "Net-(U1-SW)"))
 (segment (start 128.3 92.05) (end 128.3 91.1) (width 0.25) (layer "F.Cu") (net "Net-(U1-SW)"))
 (segment (start 130 92.25) (end 128.5 92.25) (width 0.25) (layer "F.Cu") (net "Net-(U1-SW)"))
 (segment (start 129.5 89.5) (end 129.5 88.25) (width 0.25) (layer "F.Cu") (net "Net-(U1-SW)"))
 (segment (start 130.25 96.5) (end 130.25 92.5) (width 0.25) (layer "F.Cu") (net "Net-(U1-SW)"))
 (segment (start 128.3 91.1) (end 128.3 90.7) (width 0.25) (layer "F.Cu") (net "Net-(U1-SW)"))
 (segment (start 128.3 90.7) (end 129.5 89.5) (width 0.25) (layer "F.Cu") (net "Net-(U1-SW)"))
 (segment (start 126 97.65) (end 126.85 97.65) (width 0.25) (layer "F.Cu") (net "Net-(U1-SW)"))
 (segment (start 128.5 92.25) (end 128.3 92.05) (width 0.25) (layer "F.Cu") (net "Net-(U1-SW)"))
 (segment (start 126.85 97.65) (end 127.75 96.75) (width 0.25) (layer "F.Cu") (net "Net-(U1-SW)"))
 (segment (start 127.35 91.1) (end 127.5 90.95) (width 0.25) (layer "F.Cu") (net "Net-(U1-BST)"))
 (segment (start 127.5 89.41) (end 128.66 88.25) (width 0.25) (layer "F.Cu") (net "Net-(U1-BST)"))
 (segment (start 127.5 90.95) (end 127.5 89.41) (width 0.25) (layer "F.Cu") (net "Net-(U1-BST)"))
 (segment (start 130.25 85.5) (end 130.25 86.5) (width 0.25) (layer "F.Cu") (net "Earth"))
 (segment (start 135 91.28) (end 135 92.5) (width 0.25) (layer "F.Cu") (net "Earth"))
 (segment (start 133.415 92.415) (end 132.165 92.415) (width 0.25) (layer "F.Cu") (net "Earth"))
 (segment (start 132.165 92.415) (end 131.75 92) (width 0.25) (layer "F.Cu") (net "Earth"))
 (segment (start 136.34 98) (end 137.5 98) (width 0.25) (layer "F.Cu") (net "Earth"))
 (segment (start 125.75 85) (end 122.75 85) (width 0.25) (layer "F.Cu") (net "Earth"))
 (segment (start 129.25 91.1) (end 129.25 90.682) (width 0.25) (layer "F.Cu") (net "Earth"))
 (segment (start 134.75 92.75) (end 133.75 92.75) (width 0.25) (layer "F.Cu") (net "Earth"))
 (segment (start 129.25 91.1) (end 130.15 91.1) (width 0.25) (layer "F.Cu") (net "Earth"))
 (segment (start 119.5 101.5) (end 121 100) (width 0.25) (layer "F.Cu") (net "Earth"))
 (segment (start 130 85.25) (end 130.25 85.5) (width 0.25) (layer "F.Cu") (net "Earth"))
 (segment (start 130.15 91.1) (end 130.25 91) (width 0.25) (layer "F.Cu") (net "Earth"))
 (segment (start 119.728 89.662) (end 119.728 86.272) (width 0.25) (layer "F.Cu") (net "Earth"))
 (segment (start 133.75 92.75) (end 133.415 92.415) (width 0.25) (layer "F.Cu") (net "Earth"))
 (segment (start 122.75 85) (end 121 85) (width 0.25) (layer "F.Cu") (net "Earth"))
 (segment (start 135 92.5) (end 134.75 92.75) (width 0.25) (layer "F.Cu") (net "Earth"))
 (segment (start 134.125 86.5) (end 134.125 85.262653) (width 0.25) (layer "F.Cu") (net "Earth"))
 (segment (start 119.728 86.272) (end 121 85) (width 0.25) (layer "F.Cu") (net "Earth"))
 (via (at 130.25 86.5) (size 0.8) (drill 0.4) (layers "F.Cu" "B.Cu") (free yes) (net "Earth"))
 (via (at 134.125 85.262653) (size 0.8) (drill 0.4) (layers "F.Cu" "B.Cu") (free yes) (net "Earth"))
 (via (at 130.25 91) (size 0.8) (drill 0.4) (layers "F.Cu" "B.Cu") (free yes) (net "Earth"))
 (via (at 131.75 92) (size 0.8) (drill 0.4) (layers "F.Cu" "B.Cu") (free yes) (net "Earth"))
 (via (at 121 85) (size 0.8) (drill 0.4) (layers "F.Cu" "B.Cu") (free yes) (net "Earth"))
 (via (at 137.5 98) (size 0.8) (drill 0.4) (layers "F.Cu" "B.Cu") (free yes) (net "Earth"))
 (via (at 121 100) (size 0.8) (drill 0.4) (layers "F.Cu" "B.Cu") (free yes) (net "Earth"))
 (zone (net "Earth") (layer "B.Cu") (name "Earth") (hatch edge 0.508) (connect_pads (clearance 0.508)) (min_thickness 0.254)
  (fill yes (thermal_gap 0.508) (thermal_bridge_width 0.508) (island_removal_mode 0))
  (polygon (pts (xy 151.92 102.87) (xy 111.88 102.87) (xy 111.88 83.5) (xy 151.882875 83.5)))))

